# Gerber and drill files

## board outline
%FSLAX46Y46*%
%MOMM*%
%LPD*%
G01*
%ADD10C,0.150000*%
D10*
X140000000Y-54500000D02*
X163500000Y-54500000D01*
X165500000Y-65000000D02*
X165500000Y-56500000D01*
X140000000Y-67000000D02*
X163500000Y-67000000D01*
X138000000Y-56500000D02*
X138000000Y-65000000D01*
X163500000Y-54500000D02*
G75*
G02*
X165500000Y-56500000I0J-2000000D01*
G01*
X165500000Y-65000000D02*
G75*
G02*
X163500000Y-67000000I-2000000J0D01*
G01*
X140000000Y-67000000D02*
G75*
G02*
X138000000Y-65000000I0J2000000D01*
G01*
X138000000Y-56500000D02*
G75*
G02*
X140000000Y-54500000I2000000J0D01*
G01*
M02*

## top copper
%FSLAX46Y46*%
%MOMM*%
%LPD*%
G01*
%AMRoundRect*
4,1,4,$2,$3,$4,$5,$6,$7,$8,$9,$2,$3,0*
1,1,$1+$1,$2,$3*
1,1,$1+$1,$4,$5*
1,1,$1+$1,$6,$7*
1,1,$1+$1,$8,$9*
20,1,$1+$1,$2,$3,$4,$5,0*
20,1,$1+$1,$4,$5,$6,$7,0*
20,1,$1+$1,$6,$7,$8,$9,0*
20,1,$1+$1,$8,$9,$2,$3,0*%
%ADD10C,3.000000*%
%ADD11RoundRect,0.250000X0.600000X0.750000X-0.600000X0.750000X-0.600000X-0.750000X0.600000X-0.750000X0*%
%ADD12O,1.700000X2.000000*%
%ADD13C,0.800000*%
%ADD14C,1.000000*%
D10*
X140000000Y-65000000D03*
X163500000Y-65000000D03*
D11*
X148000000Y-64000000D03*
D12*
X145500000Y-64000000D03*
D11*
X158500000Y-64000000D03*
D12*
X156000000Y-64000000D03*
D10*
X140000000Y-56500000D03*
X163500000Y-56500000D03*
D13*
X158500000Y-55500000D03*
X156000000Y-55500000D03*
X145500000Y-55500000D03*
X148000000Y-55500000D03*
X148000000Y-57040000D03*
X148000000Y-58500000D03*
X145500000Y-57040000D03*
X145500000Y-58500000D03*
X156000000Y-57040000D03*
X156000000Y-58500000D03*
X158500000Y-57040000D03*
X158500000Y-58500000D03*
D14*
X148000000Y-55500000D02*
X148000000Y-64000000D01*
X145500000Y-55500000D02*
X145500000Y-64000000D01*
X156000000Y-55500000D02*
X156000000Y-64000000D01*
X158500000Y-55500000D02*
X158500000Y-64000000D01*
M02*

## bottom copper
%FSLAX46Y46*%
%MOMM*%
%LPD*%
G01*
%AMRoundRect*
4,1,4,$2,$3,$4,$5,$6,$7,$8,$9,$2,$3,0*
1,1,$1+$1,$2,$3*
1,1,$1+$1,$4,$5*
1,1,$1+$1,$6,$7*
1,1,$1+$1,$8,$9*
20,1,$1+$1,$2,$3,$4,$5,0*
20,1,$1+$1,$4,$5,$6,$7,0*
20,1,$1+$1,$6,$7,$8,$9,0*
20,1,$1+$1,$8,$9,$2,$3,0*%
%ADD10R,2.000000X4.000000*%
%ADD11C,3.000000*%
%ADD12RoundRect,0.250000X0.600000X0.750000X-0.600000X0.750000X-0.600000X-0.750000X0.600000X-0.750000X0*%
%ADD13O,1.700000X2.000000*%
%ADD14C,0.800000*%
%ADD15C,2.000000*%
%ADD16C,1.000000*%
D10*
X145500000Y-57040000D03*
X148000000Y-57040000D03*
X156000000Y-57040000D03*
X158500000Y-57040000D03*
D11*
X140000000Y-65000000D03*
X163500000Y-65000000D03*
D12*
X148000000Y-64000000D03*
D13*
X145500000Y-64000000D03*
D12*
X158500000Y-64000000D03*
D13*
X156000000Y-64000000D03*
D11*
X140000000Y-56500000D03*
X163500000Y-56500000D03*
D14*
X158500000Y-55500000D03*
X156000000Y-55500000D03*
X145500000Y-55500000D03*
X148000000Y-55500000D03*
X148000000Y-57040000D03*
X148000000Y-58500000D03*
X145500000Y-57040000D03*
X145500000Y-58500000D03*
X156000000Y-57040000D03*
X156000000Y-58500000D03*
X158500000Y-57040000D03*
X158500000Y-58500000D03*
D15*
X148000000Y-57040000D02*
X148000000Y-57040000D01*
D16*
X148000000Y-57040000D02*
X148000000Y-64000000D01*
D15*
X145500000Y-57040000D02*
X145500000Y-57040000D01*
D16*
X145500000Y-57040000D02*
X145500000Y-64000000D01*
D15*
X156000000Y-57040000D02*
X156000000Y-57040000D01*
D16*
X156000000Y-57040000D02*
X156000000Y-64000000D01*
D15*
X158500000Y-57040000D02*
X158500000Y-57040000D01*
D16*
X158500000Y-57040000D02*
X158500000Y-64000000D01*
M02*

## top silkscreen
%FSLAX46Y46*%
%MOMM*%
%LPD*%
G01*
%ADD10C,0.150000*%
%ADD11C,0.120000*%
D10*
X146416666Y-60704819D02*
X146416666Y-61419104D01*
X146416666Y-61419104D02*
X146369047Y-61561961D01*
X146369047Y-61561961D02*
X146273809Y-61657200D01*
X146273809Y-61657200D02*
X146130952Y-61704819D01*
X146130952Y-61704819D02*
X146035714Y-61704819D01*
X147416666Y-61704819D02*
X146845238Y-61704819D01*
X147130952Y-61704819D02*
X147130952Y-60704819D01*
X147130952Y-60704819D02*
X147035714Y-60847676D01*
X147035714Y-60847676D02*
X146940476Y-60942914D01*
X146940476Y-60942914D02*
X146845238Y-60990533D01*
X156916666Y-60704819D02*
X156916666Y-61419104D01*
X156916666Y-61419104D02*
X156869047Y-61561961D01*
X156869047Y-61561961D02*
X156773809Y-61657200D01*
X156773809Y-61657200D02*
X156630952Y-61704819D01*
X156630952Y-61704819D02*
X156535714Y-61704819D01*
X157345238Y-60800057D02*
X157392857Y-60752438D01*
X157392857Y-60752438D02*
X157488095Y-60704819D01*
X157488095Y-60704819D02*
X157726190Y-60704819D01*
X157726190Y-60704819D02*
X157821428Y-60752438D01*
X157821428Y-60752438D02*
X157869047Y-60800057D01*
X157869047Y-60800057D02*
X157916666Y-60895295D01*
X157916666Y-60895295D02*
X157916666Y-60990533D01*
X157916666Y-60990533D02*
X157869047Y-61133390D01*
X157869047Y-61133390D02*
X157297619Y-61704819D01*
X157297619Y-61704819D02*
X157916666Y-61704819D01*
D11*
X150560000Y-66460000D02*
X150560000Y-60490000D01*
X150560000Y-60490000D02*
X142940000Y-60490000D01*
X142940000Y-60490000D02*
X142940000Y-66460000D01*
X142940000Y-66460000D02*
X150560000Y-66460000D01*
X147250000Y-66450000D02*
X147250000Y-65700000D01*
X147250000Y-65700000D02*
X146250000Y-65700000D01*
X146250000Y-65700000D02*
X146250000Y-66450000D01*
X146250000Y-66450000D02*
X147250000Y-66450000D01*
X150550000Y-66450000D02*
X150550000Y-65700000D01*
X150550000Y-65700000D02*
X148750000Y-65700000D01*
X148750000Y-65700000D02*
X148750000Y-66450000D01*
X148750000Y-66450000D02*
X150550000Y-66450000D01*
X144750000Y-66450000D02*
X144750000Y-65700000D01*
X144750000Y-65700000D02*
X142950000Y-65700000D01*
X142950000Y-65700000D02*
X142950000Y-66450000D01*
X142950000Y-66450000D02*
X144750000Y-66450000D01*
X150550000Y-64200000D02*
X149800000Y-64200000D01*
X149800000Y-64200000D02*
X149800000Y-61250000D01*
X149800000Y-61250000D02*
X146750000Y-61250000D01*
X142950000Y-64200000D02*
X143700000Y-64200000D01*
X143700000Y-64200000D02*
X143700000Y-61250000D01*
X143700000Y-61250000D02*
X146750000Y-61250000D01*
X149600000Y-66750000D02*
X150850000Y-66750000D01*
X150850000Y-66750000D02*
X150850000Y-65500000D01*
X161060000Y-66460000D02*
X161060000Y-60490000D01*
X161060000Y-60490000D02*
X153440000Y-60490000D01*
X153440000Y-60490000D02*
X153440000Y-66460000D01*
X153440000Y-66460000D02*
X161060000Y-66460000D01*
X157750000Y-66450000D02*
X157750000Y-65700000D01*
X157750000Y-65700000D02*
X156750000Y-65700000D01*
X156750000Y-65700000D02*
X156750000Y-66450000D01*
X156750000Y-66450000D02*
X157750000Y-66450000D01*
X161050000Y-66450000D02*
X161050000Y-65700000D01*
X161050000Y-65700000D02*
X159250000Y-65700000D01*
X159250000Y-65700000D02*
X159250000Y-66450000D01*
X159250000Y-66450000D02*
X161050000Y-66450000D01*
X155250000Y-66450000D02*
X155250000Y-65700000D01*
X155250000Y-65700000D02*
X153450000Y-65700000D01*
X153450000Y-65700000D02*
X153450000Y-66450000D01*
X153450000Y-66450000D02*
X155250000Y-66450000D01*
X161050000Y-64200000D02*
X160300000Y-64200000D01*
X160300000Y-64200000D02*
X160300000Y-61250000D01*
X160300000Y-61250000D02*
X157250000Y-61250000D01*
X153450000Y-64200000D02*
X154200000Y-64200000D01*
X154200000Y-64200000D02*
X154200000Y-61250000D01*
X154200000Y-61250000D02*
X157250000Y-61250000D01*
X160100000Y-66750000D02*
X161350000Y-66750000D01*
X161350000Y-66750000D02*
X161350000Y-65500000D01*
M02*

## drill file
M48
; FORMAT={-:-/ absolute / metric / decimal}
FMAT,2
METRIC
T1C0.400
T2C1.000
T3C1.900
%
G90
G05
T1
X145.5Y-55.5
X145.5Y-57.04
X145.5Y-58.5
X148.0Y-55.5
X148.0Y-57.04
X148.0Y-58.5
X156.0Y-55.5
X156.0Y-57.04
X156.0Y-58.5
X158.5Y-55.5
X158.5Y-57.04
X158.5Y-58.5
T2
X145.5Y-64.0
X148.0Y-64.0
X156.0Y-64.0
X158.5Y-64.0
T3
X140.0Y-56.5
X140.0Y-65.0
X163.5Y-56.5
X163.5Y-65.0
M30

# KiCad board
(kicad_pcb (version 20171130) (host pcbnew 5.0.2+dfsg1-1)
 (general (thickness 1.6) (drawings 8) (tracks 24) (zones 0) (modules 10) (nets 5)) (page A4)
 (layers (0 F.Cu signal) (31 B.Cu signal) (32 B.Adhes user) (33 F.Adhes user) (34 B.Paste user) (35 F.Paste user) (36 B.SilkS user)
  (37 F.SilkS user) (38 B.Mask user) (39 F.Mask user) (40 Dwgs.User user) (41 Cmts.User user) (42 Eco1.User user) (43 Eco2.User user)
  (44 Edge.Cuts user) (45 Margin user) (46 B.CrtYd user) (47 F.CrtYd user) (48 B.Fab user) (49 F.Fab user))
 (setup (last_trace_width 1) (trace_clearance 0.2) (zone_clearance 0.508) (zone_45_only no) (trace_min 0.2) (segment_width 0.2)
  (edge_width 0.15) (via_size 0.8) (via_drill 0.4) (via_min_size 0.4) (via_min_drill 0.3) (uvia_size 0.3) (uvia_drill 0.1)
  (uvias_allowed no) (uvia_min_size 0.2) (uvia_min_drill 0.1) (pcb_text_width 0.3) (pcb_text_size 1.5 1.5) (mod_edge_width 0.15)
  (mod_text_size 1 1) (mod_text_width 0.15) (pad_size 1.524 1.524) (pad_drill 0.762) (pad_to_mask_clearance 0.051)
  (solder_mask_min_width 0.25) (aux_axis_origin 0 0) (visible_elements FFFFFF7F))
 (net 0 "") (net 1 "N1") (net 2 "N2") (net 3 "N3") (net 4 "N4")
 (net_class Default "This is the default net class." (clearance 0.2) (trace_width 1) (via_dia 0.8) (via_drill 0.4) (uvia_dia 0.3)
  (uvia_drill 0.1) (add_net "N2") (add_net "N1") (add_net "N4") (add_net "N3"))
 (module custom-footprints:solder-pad (layer B.Cu) (at 145.5 54.5)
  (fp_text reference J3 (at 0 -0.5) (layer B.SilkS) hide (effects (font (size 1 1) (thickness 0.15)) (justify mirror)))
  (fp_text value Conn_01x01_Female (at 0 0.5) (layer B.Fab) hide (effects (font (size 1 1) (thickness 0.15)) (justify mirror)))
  (pad 1 smd rect (at 0 2.54) (size 2 4) (layers B.Cu B.Paste B.Mask) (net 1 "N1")))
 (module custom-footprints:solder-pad (layer B.Cu) (at 148 54.5)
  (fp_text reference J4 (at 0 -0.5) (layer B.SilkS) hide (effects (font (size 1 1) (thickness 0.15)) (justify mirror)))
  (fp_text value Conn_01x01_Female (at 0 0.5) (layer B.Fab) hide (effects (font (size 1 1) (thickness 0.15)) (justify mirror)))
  (pad 1 smd rect (at 0 2.54) (size 2 4) (layers B.Cu B.Paste B.Mask) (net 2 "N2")))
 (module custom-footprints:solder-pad (layer B.Cu) (at 156 54.5)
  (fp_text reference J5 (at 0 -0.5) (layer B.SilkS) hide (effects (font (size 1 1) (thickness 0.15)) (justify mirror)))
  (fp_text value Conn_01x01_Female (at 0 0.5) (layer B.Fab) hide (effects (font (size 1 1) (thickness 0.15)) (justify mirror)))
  (pad 1 smd rect (at 0 2.54) (size 2 4) (layers B.Cu B.Paste B.Mask) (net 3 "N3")))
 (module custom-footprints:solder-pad (layer B.Cu) (at 158.5 54.5)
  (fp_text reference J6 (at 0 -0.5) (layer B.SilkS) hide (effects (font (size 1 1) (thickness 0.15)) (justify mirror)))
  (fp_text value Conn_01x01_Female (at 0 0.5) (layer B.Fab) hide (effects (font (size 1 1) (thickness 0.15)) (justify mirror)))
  (pad 1 smd rect (at 0 2.54) (size 2 4) (layers B.Cu B.Paste B.Mask) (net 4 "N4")))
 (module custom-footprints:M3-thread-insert (layer F.Cu) (at 139.365 65)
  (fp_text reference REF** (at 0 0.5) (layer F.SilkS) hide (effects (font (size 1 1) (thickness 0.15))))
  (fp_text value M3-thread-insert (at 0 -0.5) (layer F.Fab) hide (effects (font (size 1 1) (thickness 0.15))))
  (pad 1 thru_hole circle (at 0.635 0) (size 3 3) (drill 1.9) (layers *.Cu *.Mask)))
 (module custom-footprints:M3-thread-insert (layer F.Cu) (at 162.865 65)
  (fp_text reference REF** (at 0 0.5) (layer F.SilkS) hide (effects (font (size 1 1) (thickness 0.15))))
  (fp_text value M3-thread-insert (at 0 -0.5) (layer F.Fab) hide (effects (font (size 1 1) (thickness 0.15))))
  (pad 1 thru_hole circle (at 0.635 0) (size 3 3) (drill 1.9) (layers *.Cu *.Mask)))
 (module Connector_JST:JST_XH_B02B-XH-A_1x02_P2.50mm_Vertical (layer F.Cu) (at 148 64 180)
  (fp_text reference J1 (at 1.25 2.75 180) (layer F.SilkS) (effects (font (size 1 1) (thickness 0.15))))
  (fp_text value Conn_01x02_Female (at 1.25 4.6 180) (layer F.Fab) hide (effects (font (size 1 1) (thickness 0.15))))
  (fp_line (start -2.56 -2.46) (end -2.56 3.51) (layer F.SilkS) (width 0.12))
  (fp_line (start -2.56 3.51) (end 5.06 3.51) (layer F.SilkS) (width 0.12))
  (fp_line (start 5.06 3.51) (end 5.06 -2.46) (layer F.SilkS) (width 0.12))
  (fp_line (start 5.06 -2.46) (end -2.56 -2.46) (layer F.SilkS) (width 0.12))
  (fp_line (start 0.75 -2.45) (end 0.75 -1.7) (layer F.SilkS) (width 0.12))
  (fp_line (start 0.75 -1.7) (end 1.75 -1.7) (layer F.SilkS) (width 0.12))
  (fp_line (start 1.75 -1.7) (end 1.75 -2.45) (layer F.SilkS) (width 0.12))
  (fp_line (start 1.75 -2.45) (end 0.75 -2.45) (layer F.SilkS) (width 0.12))
  (fp_line (start -2.55 -2.45) (end -2.55 -1.7) (layer F.SilkS) (width 0.12))
  (fp_line (start -2.55 -1.7) (end -0.75 -1.7) (layer F.SilkS) (width 0.12))
  (fp_line (start -0.75 -1.7) (end -0.75 -2.45) (layer F.SilkS) (width 0.12))
  (fp_line (start -0.75 -2.45) (end -2.55 -2.45) (layer F.SilkS) (width 0.12))
  (fp_line (start 3.25 -2.45) (end 3.25 -1.7) (layer F.SilkS) (width 0.12))
  (fp_line (start 3.25 -1.7) (end 5.05 -1.7) (layer F.SilkS) (width 0.12))
  (fp_line (start 5.05 -1.7) (end 5.05 -2.45) (layer F.SilkS) (width 0.12))
  (fp_line (start 5.05 -2.45) (end 3.25 -2.45) (layer F.SilkS) (width 0.12))
  (fp_line (start -2.55 -0.2) (end -1.8 -0.2) (layer F.SilkS) (width 0.12))
  (fp_line (start -1.8 -0.2) (end -1.8 2.75) (layer F.SilkS) (width 0.12))
  (fp_line (start -1.8 2.75) (end 1.25 2.75) (layer F.SilkS) (width 0.12))
  (fp_line (start 5.05 -0.2) (end 4.3 -0.2) (layer F.SilkS) (width 0.12))
  (fp_line (start 4.3 -0.2) (end 4.3 2.75) (layer F.SilkS) (width 0.12))
  (fp_line (start 4.3 2.75) (end 1.25 2.75) (layer F.SilkS) (width 0.12))
  (fp_line (start -1.6 -2.75) (end -2.85 -2.75) (layer F.SilkS) (width 0.12))
  (fp_line (start -2.85 -2.75) (end -2.85 -1.5) (layer F.SilkS) (width 0.12))
  (pad 1 thru_hole roundrect (at 0 0 180) (size 1.7 2) (drill 1) (layers *.Cu *.Mask) (roundrect_rratio 0.147059) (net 2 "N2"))
  (pad 2 thru_hole oval (at 2.5 0 180) (size 1.7 2) (drill 1) (layers *.Cu *.Mask) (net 1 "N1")))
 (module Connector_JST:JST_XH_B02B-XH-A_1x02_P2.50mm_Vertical (layer F.Cu) (at 158.5 64 180)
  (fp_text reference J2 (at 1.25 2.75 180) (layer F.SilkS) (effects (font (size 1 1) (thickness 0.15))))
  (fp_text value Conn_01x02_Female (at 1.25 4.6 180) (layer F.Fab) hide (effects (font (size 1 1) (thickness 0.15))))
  (fp_line (start -2.56 -2.46) (end -2.56 3.51) (layer F.SilkS) (width 0.12))
  (fp_line (start -2.56 3.51) (end 5.06 3.51) (layer F.SilkS) (width 0.12))
  (fp_line (start 5.06 3.51) (end 5.06 -2.46) (layer F.SilkS) (width 0.12))
  (fp_line (start 5.06 -2.46) (end -2.56 -2.46) (layer F.SilkS) (width 0.12))
  (fp_line (start 0.75 -2.45) (end 0.75 -1.7) (layer F.SilkS) (width 0.12))
  (fp_line (start 0.75 -1.7) (end 1.75 -1.7) (layer F.SilkS) (width 0.12))
  (fp_line (start 1.75 -1.7) (end 1.75 -2.45) (layer F.SilkS) (width 0.12))
  (fp_line (start 1.75 -2.45) (end 0.75 -2.45) (layer F.SilkS) (width 0.12))
  (fp_line (start -2.55 -2.45) (end -2.55 -1.7) (layer F.SilkS) (width 0.12))
  (fp_line (start -2.55 -1.7) (end -0.75 -1.7) (layer F.SilkS) (width 0.12))
  (fp_line (start -0.75 -1.7) (end -0.75 -2.45) (layer F.SilkS) (width 0.12))
  (fp_line (start -0.75 -2.45) (end -2.55 -2.45) (layer F.SilkS) (width 0.12))
  (fp_line (start 3.25 -2.45) (end 3.25 -1.7) (layer F.SilkS) (width 0.12))
  (fp_line (start 3.25 -1.7) (end 5.05 -1.7) (layer F.SilkS) (width 0.12))
  (fp_line (start 5.05 -1.7) (end 5.05 -2.45) (layer F.SilkS) (width 0.12))
  (fp_line (start 5.05 -2.45) (end 3.25 -2.45) (layer F.SilkS) (width 0.12))
  (fp_line (start -2.55 -0.2) (end -1.8 -0.2) (layer F.SilkS) (width 0.12))
  (fp_line (start -1.8 -0.2) (end -1.8 2.75) (layer F.SilkS) (width 0.12))
  (fp_line (start -1.8 2.75) (end 1.25 2.75) (layer F.SilkS) (width 0.12))
  (fp_line (start 5.05 -0.2) (end 4.3 -0.2) (layer F.SilkS) (width 0.12))
  (fp_line (start 4.3 -0.2) (end 4.3 2.75) (layer F.SilkS) (width 0.12))
  (fp_line (start 4.3 2.75) (end 1.25 2.75) (layer F.SilkS) (width 0.12))
  (fp_line (start -1.6 -2.75) (end -2.85 -2.75) (layer F.SilkS) (width 0.12))
  (fp_line (start -2.85 -2.75) (end -2.85 -1.5) (layer F.SilkS) (width 0.12))
  (pad 1 thru_hole roundrect (at 0 0 180) (size 1.7 2) (drill 1) (layers *.Cu *.Mask) (roundrect_rratio 0.147059) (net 4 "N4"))
  (pad 2 thru_hole oval (at 2.5 0 180) (size 1.7 2) (drill 1) (layers *.Cu *.Mask) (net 3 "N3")))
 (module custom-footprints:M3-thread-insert (layer F.Cu) (at 139.365 56.5)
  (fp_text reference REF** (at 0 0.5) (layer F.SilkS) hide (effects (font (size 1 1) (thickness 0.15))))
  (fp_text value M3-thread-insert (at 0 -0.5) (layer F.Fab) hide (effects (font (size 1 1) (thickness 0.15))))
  (pad 1 thru_hole circle (at 0.635 0) (size 3 3) (drill 1.9) (layers *.Cu *.Mask)))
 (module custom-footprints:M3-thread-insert (layer F.Cu) (at 162.865 56.5)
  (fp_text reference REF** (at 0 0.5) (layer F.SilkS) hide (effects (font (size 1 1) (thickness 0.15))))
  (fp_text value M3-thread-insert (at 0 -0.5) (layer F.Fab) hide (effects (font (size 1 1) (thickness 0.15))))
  (pad 1 thru_hole circle (at 0.635 0) (size 3 3) (drill 1.9) (layers *.Cu *.Mask)))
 (gr_line (start 140 54.5) (end 163.5 54.5) (layer Edge.Cuts) (width 0.15))
 (gr_line (start 165.5 65) (end 165.5 56.5) (layer Edge.Cuts) (width 0.15))
 (gr_line (start 140 67) (end 163.5 67) (layer Edge.Cuts) (width 0.15))
 (gr_line (start 138 56.5) (end 138 65) (layer Edge.Cuts) (width 0.15))
 (gr_arc (start 163.5 56.5) (end 165.5 56.5) (angle -90) (layer Edge.Cuts) (width 0.15))
 (gr_arc (start 163.5 65) (end 163.5 67) (angle -90) (layer Edge.Cuts) (width 0.15))
 (gr_arc (start 140 65) (end 138 65) (angle -90) (layer Edge.Cuts) (width 0.15))
 (gr_arc (start 140 56.5) (end 140 54.5) (angle -90) (layer Edge.Cuts) (width 0.15))
 (via (at 158.5 55.5) (size 0.8) (drill 0.4) (layers F.Cu B.Cu) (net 4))
 (via (at 156 55.5) (size 0.8) (drill 0.4) (layers F.Cu B.Cu) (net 3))
 (via (at 145.5 55.5) (size 0.8) (drill 0.4) (layers F.Cu B.Cu) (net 1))
 (via (at 148 55.5) (size 0.8) (drill 0.4) (layers F.Cu B.Cu) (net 2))
 (segment (start 148 57.04) (end 148 57.04) (width 2) (layer B.Cu) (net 2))
 (via (at 148 57.04) (size 0.8) (drill 0.4) (layers F.Cu B.Cu) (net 2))
 (via (at 148 58.5) (size 0.8) (drill 0.4) (layers F.Cu B.Cu) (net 2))
 (segment (start 148 57.04) (end 148 64) (width 1) (layer B.Cu) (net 2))
 (segment (start 148 55.5) (end 148 64) (width 1) (layer F.Cu) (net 2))
 (segment (start 145.5 57.04) (end 145.5 57.04) (width 2) (layer B.Cu) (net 1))
 (via (at 145.5 57.04) (size 0.8) (drill 0.4) (layers F.Cu B.Cu) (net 1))
 (via (at 145.5 58.5) (size 0.8) (drill 0.4) (layers F.Cu B.Cu) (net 1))
 (segment (start 145.5 57.04) (end 145.5 64) (width 1) (layer B.Cu) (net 1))
 (segment (start 145.5 55.5) (end 145.5 64) (width 1) (layer F.Cu) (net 1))
 (segment (start 156 57.04) (end 156 57.04) (width 2) (layer B.Cu) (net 3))
 (via (at 156 57.04) (size 0.8) (drill 0.4) (layers F.Cu B.Cu) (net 3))
 (via (at 156 58.5) (size 0.8) (drill 0.4) (layers F.Cu B.Cu) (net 3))
 (segment (start 156 57.04) (end 156 64) (width 1) (layer B.Cu) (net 3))
 (segment (start 156 55.5) (end 156 64) (width 1) (layer F.Cu) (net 3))
 (segment (start 158.5 57.04) (end 158.5 57.04) (width 2) (layer B.Cu) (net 4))
 (via (at 158.5 57.04) (size 0.8) (drill 0.4) (layers F.Cu B.Cu) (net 4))
 (via (at 158.5 58.5) (size 0.8) (drill 0.4) (layers F.Cu B.Cu) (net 4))
 (segment (start 158.5 57.04) (end 158.5 64) (width 1) (layer B.Cu) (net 4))
 (segment (start 158.5 55.5) (end 158.5 64) (width 1) (layer F.Cu) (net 4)))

